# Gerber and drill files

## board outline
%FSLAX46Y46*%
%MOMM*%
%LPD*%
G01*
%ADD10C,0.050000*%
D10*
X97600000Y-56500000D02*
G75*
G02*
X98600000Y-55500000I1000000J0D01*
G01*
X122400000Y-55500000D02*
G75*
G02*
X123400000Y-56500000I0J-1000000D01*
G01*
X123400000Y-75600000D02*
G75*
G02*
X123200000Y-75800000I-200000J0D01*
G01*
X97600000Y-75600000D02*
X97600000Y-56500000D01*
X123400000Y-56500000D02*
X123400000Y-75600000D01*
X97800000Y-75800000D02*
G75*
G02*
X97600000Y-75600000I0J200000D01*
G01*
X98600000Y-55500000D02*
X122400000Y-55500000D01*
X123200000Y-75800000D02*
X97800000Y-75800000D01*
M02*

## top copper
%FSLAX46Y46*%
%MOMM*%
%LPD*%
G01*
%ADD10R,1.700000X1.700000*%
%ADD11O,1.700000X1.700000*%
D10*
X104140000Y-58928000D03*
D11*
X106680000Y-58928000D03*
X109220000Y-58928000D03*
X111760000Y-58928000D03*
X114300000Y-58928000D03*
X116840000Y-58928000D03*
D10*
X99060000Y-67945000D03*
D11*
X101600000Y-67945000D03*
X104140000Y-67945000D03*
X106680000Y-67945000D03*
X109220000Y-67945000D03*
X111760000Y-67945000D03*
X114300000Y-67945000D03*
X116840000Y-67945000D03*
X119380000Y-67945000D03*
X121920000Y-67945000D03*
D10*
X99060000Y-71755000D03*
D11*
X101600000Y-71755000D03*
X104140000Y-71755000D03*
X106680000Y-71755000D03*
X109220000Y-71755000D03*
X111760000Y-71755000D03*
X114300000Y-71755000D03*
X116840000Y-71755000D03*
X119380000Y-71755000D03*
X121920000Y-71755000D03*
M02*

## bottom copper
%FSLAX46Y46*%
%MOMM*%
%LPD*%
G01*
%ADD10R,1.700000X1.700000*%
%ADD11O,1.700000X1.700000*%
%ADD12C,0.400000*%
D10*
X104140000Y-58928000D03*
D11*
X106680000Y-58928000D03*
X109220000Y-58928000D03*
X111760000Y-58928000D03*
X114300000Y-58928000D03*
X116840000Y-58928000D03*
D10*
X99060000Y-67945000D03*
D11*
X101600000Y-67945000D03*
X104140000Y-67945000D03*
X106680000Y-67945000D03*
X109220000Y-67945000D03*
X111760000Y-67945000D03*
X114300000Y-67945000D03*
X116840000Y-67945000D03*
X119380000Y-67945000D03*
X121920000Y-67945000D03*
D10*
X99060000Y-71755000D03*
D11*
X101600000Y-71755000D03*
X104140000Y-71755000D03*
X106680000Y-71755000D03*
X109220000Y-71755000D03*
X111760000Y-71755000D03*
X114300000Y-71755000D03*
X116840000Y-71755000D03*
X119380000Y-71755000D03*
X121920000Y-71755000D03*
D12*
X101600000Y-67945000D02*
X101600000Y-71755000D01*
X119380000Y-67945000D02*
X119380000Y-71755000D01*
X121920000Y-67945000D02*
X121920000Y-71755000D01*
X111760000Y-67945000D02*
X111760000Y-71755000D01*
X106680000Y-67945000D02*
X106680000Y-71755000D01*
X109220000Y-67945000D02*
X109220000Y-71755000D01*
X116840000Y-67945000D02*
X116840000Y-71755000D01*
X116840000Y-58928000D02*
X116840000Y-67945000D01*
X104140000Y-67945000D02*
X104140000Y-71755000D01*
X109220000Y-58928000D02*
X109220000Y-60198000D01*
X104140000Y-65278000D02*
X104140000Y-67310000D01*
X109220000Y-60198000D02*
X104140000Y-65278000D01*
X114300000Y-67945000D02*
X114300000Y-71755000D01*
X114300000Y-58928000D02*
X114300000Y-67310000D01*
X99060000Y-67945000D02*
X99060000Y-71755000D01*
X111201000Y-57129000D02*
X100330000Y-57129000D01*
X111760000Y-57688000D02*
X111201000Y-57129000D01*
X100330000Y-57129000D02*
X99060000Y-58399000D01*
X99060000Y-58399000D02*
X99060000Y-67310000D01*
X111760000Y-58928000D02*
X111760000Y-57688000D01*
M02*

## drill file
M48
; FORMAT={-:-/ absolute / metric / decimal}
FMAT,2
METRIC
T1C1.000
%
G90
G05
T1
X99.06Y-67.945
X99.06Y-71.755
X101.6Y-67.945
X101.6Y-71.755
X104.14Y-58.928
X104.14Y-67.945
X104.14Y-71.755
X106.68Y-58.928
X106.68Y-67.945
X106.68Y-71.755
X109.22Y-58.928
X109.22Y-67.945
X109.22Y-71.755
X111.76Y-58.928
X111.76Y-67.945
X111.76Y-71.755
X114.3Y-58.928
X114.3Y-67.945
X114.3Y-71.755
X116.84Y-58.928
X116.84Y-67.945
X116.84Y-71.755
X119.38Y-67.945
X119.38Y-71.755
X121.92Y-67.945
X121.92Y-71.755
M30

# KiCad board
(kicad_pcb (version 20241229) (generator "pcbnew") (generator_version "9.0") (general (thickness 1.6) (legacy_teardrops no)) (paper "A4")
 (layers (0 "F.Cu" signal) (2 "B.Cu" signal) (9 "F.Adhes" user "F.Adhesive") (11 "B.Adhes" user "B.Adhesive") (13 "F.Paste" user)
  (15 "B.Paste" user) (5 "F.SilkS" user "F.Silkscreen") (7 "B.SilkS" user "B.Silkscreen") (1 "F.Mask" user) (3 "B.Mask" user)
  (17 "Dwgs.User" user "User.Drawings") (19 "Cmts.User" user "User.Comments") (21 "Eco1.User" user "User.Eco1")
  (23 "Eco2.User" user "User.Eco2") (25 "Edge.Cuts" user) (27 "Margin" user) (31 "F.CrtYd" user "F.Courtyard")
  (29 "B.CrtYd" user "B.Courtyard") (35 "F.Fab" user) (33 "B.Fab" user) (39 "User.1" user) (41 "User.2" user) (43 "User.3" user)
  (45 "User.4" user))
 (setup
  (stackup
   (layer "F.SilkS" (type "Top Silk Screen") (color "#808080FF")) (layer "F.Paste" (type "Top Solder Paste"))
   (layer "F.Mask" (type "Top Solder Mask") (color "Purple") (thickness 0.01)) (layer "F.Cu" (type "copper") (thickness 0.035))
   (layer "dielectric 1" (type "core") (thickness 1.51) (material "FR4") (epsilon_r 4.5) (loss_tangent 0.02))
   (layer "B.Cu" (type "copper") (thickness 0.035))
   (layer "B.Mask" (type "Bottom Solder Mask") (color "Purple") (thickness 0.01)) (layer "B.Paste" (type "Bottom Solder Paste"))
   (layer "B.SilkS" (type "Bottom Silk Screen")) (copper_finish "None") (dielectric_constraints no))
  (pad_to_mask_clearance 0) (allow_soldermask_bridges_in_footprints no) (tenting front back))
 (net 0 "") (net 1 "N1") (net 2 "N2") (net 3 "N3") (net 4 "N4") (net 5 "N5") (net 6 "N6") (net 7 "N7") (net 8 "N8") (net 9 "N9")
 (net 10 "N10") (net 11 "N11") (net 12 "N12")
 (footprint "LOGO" (layer "F.Cu") (at 104.14 64.008)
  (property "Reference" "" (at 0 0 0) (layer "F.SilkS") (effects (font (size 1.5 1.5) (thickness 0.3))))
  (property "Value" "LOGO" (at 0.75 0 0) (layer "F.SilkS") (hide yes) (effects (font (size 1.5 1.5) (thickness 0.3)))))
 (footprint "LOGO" (layer "F.Cu") (at 116.586 64.15806)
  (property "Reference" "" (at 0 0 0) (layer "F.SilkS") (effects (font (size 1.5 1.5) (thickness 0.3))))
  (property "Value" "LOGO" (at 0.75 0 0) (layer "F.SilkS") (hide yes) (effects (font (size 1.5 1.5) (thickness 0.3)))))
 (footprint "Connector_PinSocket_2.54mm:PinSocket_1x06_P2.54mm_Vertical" (layer "F.Cu") (at 104.14 58.928 90)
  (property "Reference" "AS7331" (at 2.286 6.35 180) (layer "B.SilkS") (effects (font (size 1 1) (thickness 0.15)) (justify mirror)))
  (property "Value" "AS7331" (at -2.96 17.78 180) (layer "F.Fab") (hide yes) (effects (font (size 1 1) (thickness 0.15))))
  (pad "1" thru_hole rect (at 0 0 90) (size 1.7 1.7) (drill 1) (layers "*.Cu" "*.Mask") (remove_unused_layers no) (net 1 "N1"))
  (pad "2" thru_hole oval (at 0 2.54 90) (size 1.7 1.7) (drill 1) (layers "*.Cu" "*.Mask") (remove_unused_layers no) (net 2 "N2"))
  (pad "3" thru_hole oval (at 0 5.08 90) (size 1.7 1.7) (drill 1) (layers "*.Cu" "*.Mask") (remove_unused_layers no) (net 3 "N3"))
  (pad "4" thru_hole oval (at 0 7.62 90) (size 1.7 1.7) (drill 1) (layers "*.Cu" "*.Mask") (remove_unused_layers no) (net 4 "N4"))
  (pad "5" thru_hole oval (at 0 10.16 90) (size 1.7 1.7) (drill 1) (layers "*.Cu" "*.Mask") (remove_unused_layers no) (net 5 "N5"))
  (pad "6" thru_hole oval (at 0 12.7 90) (size 1.7 1.7) (drill 1) (layers "*.Cu" "*.Mask") (remove_unused_layers no) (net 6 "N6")))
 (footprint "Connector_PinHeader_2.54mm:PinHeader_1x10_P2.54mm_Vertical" (layer "B.Cu") (at 99.06 67.945 -90)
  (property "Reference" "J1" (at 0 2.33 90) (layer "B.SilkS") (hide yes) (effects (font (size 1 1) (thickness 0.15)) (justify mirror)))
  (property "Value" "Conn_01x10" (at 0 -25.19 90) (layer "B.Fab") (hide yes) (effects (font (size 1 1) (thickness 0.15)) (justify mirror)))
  (pad "1" thru_hole rect (at 0 0 270) (size 1.7 1.7) (drill 1) (layers "*.Cu" "*.Mask") (remove_unused_layers no) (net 4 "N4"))
  (pad "2" thru_hole oval (at 0 -2.54 270) (size 1.7 1.7) (drill 1) (layers "*.Cu" "*.Mask") (remove_unused_layers no) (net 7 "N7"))
  (pad "3" thru_hole oval (at 0 -5.08 270) (size 1.7 1.7) (drill 1) (layers "*.Cu" "*.Mask") (remove_unused_layers no) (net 3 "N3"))
  (pad "4" thru_hole oval (at 0 -7.62 270) (size 1.7 1.7) (drill 1) (layers "*.Cu" "*.Mask") (remove_unused_layers no) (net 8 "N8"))
  (pad "5" thru_hole oval (at 0 -10.16 270) (size 1.7 1.7) (drill 1) (layers "*.Cu" "*.Mask") (remove_unused_layers no) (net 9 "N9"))
  (pad "6" thru_hole oval (at 0 -12.7 270) (size 1.7 1.7) (drill 1) (layers "*.Cu" "*.Mask") (remove_unused_layers no) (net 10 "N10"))
  (pad "7" thru_hole oval (at 0 -15.24 270) (size 1.7 1.7) (drill 1) (layers "*.Cu" "*.Mask") (remove_unused_layers no) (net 5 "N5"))
  (pad "8" thru_hole oval (at 0 -17.78 270) (size 1.7 1.7) (drill 1) (layers "*.Cu" "*.Mask") (remove_unused_layers no) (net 6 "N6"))
  (pad "9" thru_hole oval (at 0 -20.32 270) (size 1.7 1.7) (drill 1) (layers "*.Cu" "*.Mask") (remove_unused_layers no) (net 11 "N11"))
  (pad "10" thru_hole oval (at 0 -22.86 270) (size 1.7 1.7) (drill 1) (layers "*.Cu" "*.Mask") (remove_unused_layers no) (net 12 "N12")))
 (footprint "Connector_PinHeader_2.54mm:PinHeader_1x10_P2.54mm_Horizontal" (layer "B.Cu") (at 99.06 71.755 -90)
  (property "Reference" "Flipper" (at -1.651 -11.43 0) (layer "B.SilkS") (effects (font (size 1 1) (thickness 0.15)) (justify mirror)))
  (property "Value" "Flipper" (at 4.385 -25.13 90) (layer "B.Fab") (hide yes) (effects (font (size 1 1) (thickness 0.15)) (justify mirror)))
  (pad "1" thru_hole rect (at 0 0 270) (size 1.7 1.7) (drill 1) (layers "*.Cu" "*.Mask") (remove_unused_layers no) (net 4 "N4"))
  (pad "2" thru_hole oval (at 0 -2.54 270) (size 1.7 1.7) (drill 1) (layers "*.Cu" "*.Mask") (remove_unused_layers no) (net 7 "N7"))
  (pad "3" thru_hole oval (at 0 -5.08 270) (size 1.7 1.7) (drill 1) (layers "*.Cu" "*.Mask") (remove_unused_layers no) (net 3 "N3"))
  (pad "4" thru_hole oval (at 0 -7.62 270) (size 1.7 1.7) (drill 1) (layers "*.Cu" "*.Mask") (remove_unused_layers no) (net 8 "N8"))
  (pad "5" thru_hole oval (at 0 -10.16 270) (size 1.7 1.7) (drill 1) (layers "*.Cu" "*.Mask") (remove_unused_layers no) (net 9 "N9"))
  (pad "6" thru_hole oval (at 0 -12.7 270) (size 1.7 1.7) (drill 1) (layers "*.Cu" "*.Mask") (remove_unused_layers no) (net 10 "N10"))
  (pad "7" thru_hole oval (at 0 -15.24 270) (size 1.7 1.7) (drill 1) (layers "*.Cu" "*.Mask") (remove_unused_layers no) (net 5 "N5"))
  (pad "8" thru_hole oval (at 0 -17.78 270) (size 1.7 1.7) (drill 1) (layers "*.Cu" "*.Mask") (remove_unused_layers no) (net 6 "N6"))
  (pad "9" thru_hole oval (at 0 -20.32 270) (size 1.7 1.7) (drill 1) (layers "*.Cu" "*.Mask") (remove_unused_layers no) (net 11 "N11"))
  (pad "10" thru_hole oval (at 0 -22.86 270) (size 1.7 1.7) (drill 1) (layers "*.Cu" "*.Mask") (remove_unused_layers no) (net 12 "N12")))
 (gr_arc (start 97.6 56.5) (mid 97.892893 55.792893) (end 98.6 55.5) (stroke (width 0.05) (type default)) (layer "Edge.Cuts"))
 (gr_arc (start 122.4 55.5) (mid 123.107107 55.792893) (end 123.4 56.5) (stroke (width 0.05) (type default)) (layer "Edge.Cuts"))
 (gr_arc (start 123.4 75.6) (mid 123.341421 75.741421) (end 123.2 75.8) (stroke (width 0.05) (type default)) (layer "Edge.Cuts"))
 (gr_line (start 97.6 75.6) (end 97.6 56.5) (stroke (width 0.05) (type default)) (layer "Edge.Cuts"))
 (gr_line (start 123.4 56.5) (end 123.4 75.6) (stroke (width 0.05) (type default)) (layer "Edge.Cuts"))
 (gr_arc (start 97.8 75.8) (mid 97.658579 75.741421) (end 97.6 75.6) (stroke (width 0.05) (type default)) (layer "Edge.Cuts"))
 (gr_line (start 98.6 55.5) (end 122.4 55.5) (stroke (width 0.05) (type default)) (layer "Edge.Cuts"))
 (gr_line (start 123.2 75.8) (end 97.8 75.8) (stroke (width 0.05) (type default)) (layer "Edge.Cuts"))
 (segment (start 101.6 67.945) (end 101.6 71.755) (width 0.4) (layer "B.Cu") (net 7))
 (segment (start 119.38 67.945) (end 119.38 71.755) (width 0.4) (layer "B.Cu") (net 11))
 (segment (start 121.92 67.945) (end 121.92 71.755) (width 0.4) (layer "B.Cu") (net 12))
 (segment (start 111.76 67.945) (end 111.76 71.755) (width 0.4) (layer "B.Cu") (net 10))
 (segment (start 106.68 67.945) (end 106.68 71.755) (width 0.4) (layer "B.Cu") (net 8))
 (segment (start 109.22 67.945) (end 109.22 71.755) (width 0.4) (layer "B.Cu") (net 9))
 (segment (start 116.84 67.945) (end 116.84 71.755) (width 0.4) (layer "B.Cu") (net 6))
 (segment (start 116.84 58.928) (end 116.84 67.945) (width 0.4) (layer "B.Cu") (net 6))
 (segment (start 104.14 67.945) (end 104.14 71.755) (width 0.4) (layer "B.Cu") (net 3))
 (segment (start 109.22 58.928) (end 109.22 60.198) (width 0.4) (layer "B.Cu") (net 3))
 (segment (start 104.14 65.278) (end 104.14 67.31) (width 0.4) (layer "B.Cu") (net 3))
 (segment (start 109.22 60.198) (end 104.14 65.278) (width 0.4) (layer "B.Cu") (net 3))
 (segment (start 114.3 67.945) (end 114.3 71.755) (width 0.4) (layer "B.Cu") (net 5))
 (segment (start 114.3 58.928) (end 114.3 67.31) (width 0.4) (layer "B.Cu") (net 5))
 (segment (start 99.06 67.945) (end 99.06 71.755) (width 0.4) (layer "B.Cu") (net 4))
 (segment (start 111.201 57.129) (end 100.33 57.129) (width 0.4) (layer "B.Cu") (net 4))
 (segment (start 111.76 57.688) (end 111.201 57.129) (width 0.4) (layer "B.Cu") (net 4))
 (segment (start 100.33 57.129) (end 99.06 58.399) (width 0.4) (layer "B.Cu") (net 4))
 (segment (start 99.06 58.399) (end 99.06 67.31) (width 0.4) (layer "B.Cu") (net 4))
 (segment (start 111.76 58.928) (end 111.76 57.688) (width 0.4) (layer "B.Cu") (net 4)))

